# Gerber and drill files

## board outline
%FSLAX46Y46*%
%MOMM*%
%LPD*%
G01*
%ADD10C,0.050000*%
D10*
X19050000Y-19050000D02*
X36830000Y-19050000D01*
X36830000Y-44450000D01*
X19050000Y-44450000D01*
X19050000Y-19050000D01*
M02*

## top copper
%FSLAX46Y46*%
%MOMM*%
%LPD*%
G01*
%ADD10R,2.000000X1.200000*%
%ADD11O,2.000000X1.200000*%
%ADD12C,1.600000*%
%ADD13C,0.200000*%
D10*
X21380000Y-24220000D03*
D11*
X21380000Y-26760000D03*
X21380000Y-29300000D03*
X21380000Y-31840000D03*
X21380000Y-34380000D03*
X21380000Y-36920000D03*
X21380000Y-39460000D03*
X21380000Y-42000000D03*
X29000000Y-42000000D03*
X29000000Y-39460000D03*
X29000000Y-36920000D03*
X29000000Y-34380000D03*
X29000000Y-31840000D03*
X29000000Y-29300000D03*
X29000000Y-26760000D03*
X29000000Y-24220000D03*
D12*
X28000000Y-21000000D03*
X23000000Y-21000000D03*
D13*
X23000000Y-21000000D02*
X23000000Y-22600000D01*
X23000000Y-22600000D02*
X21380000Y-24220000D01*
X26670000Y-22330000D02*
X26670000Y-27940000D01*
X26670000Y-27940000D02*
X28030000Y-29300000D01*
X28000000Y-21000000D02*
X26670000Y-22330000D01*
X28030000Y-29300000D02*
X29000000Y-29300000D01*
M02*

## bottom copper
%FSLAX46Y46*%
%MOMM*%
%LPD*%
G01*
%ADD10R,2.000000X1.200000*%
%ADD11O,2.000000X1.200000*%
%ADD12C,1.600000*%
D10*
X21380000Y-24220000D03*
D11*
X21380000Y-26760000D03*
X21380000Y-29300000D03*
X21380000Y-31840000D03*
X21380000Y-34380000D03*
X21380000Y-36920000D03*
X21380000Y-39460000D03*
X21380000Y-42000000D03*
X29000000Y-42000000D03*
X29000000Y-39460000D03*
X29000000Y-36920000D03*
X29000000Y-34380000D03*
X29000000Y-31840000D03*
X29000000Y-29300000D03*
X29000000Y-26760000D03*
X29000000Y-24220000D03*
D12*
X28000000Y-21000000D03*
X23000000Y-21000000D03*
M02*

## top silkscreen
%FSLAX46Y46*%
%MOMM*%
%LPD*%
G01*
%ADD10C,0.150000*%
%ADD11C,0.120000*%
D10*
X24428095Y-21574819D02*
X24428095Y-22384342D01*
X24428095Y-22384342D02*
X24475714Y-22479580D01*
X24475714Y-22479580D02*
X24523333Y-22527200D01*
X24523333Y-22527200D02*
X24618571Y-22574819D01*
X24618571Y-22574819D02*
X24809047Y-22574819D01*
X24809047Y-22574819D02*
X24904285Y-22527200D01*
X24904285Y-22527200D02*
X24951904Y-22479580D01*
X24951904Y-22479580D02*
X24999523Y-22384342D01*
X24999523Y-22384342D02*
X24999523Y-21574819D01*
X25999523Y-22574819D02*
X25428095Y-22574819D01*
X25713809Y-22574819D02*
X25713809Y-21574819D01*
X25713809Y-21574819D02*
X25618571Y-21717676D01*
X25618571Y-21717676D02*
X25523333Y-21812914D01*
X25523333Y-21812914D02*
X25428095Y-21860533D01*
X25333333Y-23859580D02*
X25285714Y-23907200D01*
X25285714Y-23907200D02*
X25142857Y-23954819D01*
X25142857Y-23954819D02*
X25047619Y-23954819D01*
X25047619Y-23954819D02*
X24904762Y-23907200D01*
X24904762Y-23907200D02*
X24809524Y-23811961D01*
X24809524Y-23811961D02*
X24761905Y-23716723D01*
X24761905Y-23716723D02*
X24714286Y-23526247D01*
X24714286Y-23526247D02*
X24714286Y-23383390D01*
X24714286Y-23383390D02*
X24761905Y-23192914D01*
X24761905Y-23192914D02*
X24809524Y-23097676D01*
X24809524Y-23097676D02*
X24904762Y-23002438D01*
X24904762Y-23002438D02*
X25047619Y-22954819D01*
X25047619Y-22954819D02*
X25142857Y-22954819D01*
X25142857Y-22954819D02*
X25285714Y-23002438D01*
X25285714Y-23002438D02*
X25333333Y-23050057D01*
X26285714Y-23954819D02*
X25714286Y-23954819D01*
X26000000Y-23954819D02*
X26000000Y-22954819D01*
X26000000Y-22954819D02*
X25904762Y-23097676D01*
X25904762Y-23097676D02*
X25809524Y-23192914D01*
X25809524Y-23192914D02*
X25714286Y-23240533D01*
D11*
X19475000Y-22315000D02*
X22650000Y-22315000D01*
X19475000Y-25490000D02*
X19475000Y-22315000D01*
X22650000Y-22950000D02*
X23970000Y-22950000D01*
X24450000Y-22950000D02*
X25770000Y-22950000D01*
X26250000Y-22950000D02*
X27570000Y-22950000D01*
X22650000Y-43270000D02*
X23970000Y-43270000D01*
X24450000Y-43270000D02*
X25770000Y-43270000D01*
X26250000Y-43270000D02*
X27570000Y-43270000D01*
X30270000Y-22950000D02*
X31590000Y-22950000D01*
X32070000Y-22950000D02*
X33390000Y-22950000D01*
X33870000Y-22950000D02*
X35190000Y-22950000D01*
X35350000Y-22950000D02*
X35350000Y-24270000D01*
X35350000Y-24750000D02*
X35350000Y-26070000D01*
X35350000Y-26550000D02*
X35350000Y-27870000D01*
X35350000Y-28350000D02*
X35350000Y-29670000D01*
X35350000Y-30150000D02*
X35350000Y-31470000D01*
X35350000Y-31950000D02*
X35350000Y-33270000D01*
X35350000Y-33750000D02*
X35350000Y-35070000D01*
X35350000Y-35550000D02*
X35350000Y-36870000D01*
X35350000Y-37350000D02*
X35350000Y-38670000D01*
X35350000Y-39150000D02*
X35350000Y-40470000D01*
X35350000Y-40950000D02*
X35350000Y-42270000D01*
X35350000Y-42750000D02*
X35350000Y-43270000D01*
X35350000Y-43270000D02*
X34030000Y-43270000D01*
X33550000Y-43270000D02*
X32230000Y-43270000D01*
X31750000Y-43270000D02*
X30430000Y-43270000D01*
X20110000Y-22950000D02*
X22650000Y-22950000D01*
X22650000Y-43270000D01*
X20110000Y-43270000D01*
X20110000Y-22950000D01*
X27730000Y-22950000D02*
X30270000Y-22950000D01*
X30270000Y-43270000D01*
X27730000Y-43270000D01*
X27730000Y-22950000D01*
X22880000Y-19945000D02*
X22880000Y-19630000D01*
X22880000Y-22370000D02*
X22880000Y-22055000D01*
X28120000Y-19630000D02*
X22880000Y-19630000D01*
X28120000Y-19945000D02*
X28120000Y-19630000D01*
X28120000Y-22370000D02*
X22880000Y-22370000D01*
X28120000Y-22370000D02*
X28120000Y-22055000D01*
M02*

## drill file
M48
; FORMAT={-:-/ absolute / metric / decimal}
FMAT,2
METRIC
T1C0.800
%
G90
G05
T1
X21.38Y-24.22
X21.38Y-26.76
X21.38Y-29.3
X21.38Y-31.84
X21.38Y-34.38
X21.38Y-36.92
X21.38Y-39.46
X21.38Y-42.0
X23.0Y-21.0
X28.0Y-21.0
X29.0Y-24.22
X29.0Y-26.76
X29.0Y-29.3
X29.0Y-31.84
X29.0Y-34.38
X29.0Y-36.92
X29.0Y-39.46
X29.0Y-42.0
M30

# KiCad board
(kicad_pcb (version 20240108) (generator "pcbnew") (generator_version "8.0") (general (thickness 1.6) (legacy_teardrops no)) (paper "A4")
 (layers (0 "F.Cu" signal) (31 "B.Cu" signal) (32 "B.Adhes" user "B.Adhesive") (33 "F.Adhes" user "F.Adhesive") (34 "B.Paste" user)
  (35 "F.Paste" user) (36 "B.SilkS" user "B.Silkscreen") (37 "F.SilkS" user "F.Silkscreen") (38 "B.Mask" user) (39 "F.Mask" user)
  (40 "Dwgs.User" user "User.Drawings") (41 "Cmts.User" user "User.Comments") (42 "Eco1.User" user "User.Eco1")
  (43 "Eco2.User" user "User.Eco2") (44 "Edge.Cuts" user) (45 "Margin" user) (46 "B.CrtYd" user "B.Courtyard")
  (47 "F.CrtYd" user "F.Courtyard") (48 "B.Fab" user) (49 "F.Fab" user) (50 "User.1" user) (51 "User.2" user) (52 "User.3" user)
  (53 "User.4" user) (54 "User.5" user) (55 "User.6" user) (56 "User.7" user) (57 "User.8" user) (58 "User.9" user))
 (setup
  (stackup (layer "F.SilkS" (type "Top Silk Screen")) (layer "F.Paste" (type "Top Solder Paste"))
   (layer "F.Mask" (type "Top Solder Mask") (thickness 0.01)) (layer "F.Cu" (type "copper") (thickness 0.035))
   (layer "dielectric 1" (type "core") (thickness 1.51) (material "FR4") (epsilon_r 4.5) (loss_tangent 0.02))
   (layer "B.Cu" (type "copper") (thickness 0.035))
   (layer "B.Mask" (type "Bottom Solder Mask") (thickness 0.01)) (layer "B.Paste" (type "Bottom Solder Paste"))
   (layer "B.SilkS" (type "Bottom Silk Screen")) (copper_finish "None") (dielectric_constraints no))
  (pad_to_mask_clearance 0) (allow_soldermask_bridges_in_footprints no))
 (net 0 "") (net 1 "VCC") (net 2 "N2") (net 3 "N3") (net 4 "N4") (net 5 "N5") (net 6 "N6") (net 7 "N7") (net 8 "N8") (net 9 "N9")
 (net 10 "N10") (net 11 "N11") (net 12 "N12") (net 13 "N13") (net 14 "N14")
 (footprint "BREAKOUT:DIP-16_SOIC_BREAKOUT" (layer "F.Cu") (at 21.38 24.22)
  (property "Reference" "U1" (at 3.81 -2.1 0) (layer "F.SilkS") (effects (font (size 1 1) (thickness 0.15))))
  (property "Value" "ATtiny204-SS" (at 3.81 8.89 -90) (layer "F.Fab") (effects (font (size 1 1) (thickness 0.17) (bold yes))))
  (fp_line (start -1.905 -1.905) (end 1.27 -1.905) (stroke (width 0.12) (type default)) (layer "F.SilkS"))
  (fp_line (start -1.905 1.27) (end -1.905 -1.905) (stroke (width 0.12) (type default)) (layer "F.SilkS"))
  (fp_line (start 1.27 -1.27) (end 6.35 -1.27) (stroke (width 0.12) (type dash)) (layer "F.SilkS"))
  (fp_line (start 1.27 19.05) (end 6.35 19.05) (stroke (width 0.12) (type dash)) (layer "F.SilkS"))
  (fp_line (start 8.89 -1.27) (end 13.97 -1.27) (stroke (width 0.12) (type dash)) (layer "F.SilkS"))
  (fp_line (start 13.97 -1.27) (end 13.97 19.05) (stroke (width 0.12) (type dash)) (layer "F.SilkS"))
  (fp_line (start 13.97 19.05) (end 8.89 19.05) (stroke (width 0.12) (type dash)) (layer "F.SilkS"))
  (fp_rect (start -1.27 -1.27) (end 1.27 19.05) (stroke (width 0.12) (type default)) (fill none) (layer "F.SilkS"))
  (fp_rect (start 6.35 -1.27) (end 8.89 19.05) (stroke (width 0.12) (type default)) (fill none) (layer "F.SilkS"))
  (pad "1" thru_hole rect (at 0 0 270) (size 1.2 2) (drill 0.8) (layers "*.Cu" "*.Mask") (remove_unused_layers no) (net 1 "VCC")
   (thermal_bridge_angle 45))
  (pad "2" thru_hole oval (at 0 2.54 270) (size 1.2 2) (drill 0.8) (layers "*.Cu" "*.Mask") (remove_unused_layers no) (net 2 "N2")
   (thermal_bridge_angle 45))
  (pad "3" thru_hole oval (at 0 5.08 270) (size 1.2 2) (drill 0.8) (layers "*.Cu" "*.Mask") (remove_unused_layers no) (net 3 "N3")
   (thermal_bridge_angle 45))
  (pad "4" thru_hole oval (at 0 7.62 270) (size 1.2 2) (drill 0.8) (layers "*.Cu" "*.Mask") (remove_unused_layers no) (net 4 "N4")
   (thermal_bridge_angle 45))
  (pad "5" thru_hole oval (at 0 10.16 270) (size 1.2 2) (drill 0.8) (layers "*.Cu" "*.Mask") (remove_unused_layers no) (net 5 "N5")
   (thermal_bridge_angle 45))
  (pad "6" thru_hole oval (at 0 12.7 270) (size 1.2 2) (drill 0.8) (layers "*.Cu" "*.Mask") (remove_unused_layers no) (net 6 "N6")
   (thermal_bridge_angle 45))
  (pad "7" thru_hole oval (at 0 15.24 270) (size 1.2 2) (drill 0.8) (layers "*.Cu" "*.Mask") (remove_unused_layers no) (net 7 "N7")
   (thermal_bridge_angle 45))
  (pad "8" thru_hole oval (at 0 17.78 270) (size 1.2 2) (drill 0.8) (layers "*.Cu" "*.Mask") (remove_unused_layers no) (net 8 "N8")
   (thermal_bridge_angle 45))
  (pad "9" thru_hole oval (at 7.62 17.78 270) (size 1.2 2) (drill 0.8) (layers "*.Cu" "*.Mask") (remove_unused_layers no) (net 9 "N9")
   (thermal_bridge_angle 45))
  (pad "10" thru_hole oval (at 7.62 15.24 270) (size 1.2 2) (drill 0.8) (layers "*.Cu" "*.Mask") (remove_unused_layers no) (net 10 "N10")
   (thermal_bridge_angle 45))
  (pad "11" thru_hole oval (at 7.62 12.7 270) (size 1.2 2) (drill 0.8) (layers "*.Cu" "*.Mask") (remove_unused_layers no) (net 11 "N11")
   (thermal_bridge_angle 45))
  (pad "12" thru_hole oval (at 7.62 10.16 270) (size 1.2 2) (drill 0.8) (layers "*.Cu" "*.Mask") (remove_unused_layers no) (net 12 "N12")
   (thermal_bridge_angle 45))
  (pad "13" thru_hole oval (at 7.62 7.62 270) (size 1.2 2) (drill 0.8) (layers "*.Cu" "*.Mask") (remove_unused_layers no) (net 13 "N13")
   (thermal_bridge_angle 45))
  (pad "14" thru_hole oval (at 7.62 5.08 270) (size 1.2 2) (drill 0.8) (layers "*.Cu" "*.Mask") (remove_unused_layers no) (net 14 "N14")
   (thermal_bridge_angle 45))
  (pad "15" thru_hole oval (at 7.62 2.54 270) (size 1.2 2) (drill 0.8) (layers "*.Cu" "*.Mask") (remove_unused_layers no)
   (thermal_bridge_angle 45))
  (pad "16" thru_hole oval (at 7.62 0 270) (size 1.2 2) (drill 0.8) (layers "*.Cu" "*.Mask") (remove_unused_layers no)
   (thermal_bridge_angle 45)))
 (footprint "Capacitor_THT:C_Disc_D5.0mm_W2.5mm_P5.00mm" (layer "F.Cu") (at 28 21 180)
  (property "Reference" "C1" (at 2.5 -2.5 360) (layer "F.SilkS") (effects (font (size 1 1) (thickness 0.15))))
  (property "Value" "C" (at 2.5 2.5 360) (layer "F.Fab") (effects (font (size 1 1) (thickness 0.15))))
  (fp_line (start 5.12 1.055) (end 5.12 1.37) (stroke (width 0.12) (type solid)) (layer "F.SilkS"))
  (fp_line (start 5.12 -1.37) (end 5.12 -1.055) (stroke (width 0.12) (type solid)) (layer "F.SilkS"))
  (fp_line (start -0.12 1.37) (end 5.12 1.37) (stroke (width 0.12) (type solid)) (layer "F.SilkS"))
  (fp_line (start -0.12 1.055) (end -0.12 1.37) (stroke (width 0.12) (type solid)) (layer "F.SilkS"))
  (fp_line (start -0.12 -1.37) (end 5.12 -1.37) (stroke (width 0.12) (type solid)) (layer "F.SilkS"))
  (fp_line (start -0.12 -1.37) (end -0.12 -1.055) (stroke (width 0.12) (type solid)) (layer "F.SilkS"))
  (pad "1" thru_hole circle (at 0 0 180) (size 1.6 1.6) (drill 0.8) (layers "*.Cu" "*.Mask") (remove_unused_layers no) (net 14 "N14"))
  (pad "2" thru_hole circle (at 5 0 180) (size 1.6 1.6) (drill 0.8) (layers "*.Cu" "*.Mask") (remove_unused_layers no) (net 1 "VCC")))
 (gr_rect (start 19.05 19.05) (end 36.83 44.45) (stroke (width 0.05) (type default)) (fill none) (layer "Edge.Cuts"))
 (segment (start 23 21) (end 23 22.6) (width 0.2) (layer "F.Cu") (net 1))
 (segment (start 23 22.6) (end 21.38 24.22) (width 0.2) (layer "F.Cu") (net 1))
 (segment (start 26.67 22.33) (end 26.67 27.94) (width 0.2) (layer "F.Cu") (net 14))
 (segment (start 26.67 27.94) (end 28.03 29.3) (width 0.2) (layer "F.Cu") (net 14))
 (segment (start 28 21) (end 26.67 22.33) (width 0.2) (layer "F.Cu") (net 14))
 (segment (start 28.03 29.3) (end 29 29.3) (width 0.2) (layer "F.Cu") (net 14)))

